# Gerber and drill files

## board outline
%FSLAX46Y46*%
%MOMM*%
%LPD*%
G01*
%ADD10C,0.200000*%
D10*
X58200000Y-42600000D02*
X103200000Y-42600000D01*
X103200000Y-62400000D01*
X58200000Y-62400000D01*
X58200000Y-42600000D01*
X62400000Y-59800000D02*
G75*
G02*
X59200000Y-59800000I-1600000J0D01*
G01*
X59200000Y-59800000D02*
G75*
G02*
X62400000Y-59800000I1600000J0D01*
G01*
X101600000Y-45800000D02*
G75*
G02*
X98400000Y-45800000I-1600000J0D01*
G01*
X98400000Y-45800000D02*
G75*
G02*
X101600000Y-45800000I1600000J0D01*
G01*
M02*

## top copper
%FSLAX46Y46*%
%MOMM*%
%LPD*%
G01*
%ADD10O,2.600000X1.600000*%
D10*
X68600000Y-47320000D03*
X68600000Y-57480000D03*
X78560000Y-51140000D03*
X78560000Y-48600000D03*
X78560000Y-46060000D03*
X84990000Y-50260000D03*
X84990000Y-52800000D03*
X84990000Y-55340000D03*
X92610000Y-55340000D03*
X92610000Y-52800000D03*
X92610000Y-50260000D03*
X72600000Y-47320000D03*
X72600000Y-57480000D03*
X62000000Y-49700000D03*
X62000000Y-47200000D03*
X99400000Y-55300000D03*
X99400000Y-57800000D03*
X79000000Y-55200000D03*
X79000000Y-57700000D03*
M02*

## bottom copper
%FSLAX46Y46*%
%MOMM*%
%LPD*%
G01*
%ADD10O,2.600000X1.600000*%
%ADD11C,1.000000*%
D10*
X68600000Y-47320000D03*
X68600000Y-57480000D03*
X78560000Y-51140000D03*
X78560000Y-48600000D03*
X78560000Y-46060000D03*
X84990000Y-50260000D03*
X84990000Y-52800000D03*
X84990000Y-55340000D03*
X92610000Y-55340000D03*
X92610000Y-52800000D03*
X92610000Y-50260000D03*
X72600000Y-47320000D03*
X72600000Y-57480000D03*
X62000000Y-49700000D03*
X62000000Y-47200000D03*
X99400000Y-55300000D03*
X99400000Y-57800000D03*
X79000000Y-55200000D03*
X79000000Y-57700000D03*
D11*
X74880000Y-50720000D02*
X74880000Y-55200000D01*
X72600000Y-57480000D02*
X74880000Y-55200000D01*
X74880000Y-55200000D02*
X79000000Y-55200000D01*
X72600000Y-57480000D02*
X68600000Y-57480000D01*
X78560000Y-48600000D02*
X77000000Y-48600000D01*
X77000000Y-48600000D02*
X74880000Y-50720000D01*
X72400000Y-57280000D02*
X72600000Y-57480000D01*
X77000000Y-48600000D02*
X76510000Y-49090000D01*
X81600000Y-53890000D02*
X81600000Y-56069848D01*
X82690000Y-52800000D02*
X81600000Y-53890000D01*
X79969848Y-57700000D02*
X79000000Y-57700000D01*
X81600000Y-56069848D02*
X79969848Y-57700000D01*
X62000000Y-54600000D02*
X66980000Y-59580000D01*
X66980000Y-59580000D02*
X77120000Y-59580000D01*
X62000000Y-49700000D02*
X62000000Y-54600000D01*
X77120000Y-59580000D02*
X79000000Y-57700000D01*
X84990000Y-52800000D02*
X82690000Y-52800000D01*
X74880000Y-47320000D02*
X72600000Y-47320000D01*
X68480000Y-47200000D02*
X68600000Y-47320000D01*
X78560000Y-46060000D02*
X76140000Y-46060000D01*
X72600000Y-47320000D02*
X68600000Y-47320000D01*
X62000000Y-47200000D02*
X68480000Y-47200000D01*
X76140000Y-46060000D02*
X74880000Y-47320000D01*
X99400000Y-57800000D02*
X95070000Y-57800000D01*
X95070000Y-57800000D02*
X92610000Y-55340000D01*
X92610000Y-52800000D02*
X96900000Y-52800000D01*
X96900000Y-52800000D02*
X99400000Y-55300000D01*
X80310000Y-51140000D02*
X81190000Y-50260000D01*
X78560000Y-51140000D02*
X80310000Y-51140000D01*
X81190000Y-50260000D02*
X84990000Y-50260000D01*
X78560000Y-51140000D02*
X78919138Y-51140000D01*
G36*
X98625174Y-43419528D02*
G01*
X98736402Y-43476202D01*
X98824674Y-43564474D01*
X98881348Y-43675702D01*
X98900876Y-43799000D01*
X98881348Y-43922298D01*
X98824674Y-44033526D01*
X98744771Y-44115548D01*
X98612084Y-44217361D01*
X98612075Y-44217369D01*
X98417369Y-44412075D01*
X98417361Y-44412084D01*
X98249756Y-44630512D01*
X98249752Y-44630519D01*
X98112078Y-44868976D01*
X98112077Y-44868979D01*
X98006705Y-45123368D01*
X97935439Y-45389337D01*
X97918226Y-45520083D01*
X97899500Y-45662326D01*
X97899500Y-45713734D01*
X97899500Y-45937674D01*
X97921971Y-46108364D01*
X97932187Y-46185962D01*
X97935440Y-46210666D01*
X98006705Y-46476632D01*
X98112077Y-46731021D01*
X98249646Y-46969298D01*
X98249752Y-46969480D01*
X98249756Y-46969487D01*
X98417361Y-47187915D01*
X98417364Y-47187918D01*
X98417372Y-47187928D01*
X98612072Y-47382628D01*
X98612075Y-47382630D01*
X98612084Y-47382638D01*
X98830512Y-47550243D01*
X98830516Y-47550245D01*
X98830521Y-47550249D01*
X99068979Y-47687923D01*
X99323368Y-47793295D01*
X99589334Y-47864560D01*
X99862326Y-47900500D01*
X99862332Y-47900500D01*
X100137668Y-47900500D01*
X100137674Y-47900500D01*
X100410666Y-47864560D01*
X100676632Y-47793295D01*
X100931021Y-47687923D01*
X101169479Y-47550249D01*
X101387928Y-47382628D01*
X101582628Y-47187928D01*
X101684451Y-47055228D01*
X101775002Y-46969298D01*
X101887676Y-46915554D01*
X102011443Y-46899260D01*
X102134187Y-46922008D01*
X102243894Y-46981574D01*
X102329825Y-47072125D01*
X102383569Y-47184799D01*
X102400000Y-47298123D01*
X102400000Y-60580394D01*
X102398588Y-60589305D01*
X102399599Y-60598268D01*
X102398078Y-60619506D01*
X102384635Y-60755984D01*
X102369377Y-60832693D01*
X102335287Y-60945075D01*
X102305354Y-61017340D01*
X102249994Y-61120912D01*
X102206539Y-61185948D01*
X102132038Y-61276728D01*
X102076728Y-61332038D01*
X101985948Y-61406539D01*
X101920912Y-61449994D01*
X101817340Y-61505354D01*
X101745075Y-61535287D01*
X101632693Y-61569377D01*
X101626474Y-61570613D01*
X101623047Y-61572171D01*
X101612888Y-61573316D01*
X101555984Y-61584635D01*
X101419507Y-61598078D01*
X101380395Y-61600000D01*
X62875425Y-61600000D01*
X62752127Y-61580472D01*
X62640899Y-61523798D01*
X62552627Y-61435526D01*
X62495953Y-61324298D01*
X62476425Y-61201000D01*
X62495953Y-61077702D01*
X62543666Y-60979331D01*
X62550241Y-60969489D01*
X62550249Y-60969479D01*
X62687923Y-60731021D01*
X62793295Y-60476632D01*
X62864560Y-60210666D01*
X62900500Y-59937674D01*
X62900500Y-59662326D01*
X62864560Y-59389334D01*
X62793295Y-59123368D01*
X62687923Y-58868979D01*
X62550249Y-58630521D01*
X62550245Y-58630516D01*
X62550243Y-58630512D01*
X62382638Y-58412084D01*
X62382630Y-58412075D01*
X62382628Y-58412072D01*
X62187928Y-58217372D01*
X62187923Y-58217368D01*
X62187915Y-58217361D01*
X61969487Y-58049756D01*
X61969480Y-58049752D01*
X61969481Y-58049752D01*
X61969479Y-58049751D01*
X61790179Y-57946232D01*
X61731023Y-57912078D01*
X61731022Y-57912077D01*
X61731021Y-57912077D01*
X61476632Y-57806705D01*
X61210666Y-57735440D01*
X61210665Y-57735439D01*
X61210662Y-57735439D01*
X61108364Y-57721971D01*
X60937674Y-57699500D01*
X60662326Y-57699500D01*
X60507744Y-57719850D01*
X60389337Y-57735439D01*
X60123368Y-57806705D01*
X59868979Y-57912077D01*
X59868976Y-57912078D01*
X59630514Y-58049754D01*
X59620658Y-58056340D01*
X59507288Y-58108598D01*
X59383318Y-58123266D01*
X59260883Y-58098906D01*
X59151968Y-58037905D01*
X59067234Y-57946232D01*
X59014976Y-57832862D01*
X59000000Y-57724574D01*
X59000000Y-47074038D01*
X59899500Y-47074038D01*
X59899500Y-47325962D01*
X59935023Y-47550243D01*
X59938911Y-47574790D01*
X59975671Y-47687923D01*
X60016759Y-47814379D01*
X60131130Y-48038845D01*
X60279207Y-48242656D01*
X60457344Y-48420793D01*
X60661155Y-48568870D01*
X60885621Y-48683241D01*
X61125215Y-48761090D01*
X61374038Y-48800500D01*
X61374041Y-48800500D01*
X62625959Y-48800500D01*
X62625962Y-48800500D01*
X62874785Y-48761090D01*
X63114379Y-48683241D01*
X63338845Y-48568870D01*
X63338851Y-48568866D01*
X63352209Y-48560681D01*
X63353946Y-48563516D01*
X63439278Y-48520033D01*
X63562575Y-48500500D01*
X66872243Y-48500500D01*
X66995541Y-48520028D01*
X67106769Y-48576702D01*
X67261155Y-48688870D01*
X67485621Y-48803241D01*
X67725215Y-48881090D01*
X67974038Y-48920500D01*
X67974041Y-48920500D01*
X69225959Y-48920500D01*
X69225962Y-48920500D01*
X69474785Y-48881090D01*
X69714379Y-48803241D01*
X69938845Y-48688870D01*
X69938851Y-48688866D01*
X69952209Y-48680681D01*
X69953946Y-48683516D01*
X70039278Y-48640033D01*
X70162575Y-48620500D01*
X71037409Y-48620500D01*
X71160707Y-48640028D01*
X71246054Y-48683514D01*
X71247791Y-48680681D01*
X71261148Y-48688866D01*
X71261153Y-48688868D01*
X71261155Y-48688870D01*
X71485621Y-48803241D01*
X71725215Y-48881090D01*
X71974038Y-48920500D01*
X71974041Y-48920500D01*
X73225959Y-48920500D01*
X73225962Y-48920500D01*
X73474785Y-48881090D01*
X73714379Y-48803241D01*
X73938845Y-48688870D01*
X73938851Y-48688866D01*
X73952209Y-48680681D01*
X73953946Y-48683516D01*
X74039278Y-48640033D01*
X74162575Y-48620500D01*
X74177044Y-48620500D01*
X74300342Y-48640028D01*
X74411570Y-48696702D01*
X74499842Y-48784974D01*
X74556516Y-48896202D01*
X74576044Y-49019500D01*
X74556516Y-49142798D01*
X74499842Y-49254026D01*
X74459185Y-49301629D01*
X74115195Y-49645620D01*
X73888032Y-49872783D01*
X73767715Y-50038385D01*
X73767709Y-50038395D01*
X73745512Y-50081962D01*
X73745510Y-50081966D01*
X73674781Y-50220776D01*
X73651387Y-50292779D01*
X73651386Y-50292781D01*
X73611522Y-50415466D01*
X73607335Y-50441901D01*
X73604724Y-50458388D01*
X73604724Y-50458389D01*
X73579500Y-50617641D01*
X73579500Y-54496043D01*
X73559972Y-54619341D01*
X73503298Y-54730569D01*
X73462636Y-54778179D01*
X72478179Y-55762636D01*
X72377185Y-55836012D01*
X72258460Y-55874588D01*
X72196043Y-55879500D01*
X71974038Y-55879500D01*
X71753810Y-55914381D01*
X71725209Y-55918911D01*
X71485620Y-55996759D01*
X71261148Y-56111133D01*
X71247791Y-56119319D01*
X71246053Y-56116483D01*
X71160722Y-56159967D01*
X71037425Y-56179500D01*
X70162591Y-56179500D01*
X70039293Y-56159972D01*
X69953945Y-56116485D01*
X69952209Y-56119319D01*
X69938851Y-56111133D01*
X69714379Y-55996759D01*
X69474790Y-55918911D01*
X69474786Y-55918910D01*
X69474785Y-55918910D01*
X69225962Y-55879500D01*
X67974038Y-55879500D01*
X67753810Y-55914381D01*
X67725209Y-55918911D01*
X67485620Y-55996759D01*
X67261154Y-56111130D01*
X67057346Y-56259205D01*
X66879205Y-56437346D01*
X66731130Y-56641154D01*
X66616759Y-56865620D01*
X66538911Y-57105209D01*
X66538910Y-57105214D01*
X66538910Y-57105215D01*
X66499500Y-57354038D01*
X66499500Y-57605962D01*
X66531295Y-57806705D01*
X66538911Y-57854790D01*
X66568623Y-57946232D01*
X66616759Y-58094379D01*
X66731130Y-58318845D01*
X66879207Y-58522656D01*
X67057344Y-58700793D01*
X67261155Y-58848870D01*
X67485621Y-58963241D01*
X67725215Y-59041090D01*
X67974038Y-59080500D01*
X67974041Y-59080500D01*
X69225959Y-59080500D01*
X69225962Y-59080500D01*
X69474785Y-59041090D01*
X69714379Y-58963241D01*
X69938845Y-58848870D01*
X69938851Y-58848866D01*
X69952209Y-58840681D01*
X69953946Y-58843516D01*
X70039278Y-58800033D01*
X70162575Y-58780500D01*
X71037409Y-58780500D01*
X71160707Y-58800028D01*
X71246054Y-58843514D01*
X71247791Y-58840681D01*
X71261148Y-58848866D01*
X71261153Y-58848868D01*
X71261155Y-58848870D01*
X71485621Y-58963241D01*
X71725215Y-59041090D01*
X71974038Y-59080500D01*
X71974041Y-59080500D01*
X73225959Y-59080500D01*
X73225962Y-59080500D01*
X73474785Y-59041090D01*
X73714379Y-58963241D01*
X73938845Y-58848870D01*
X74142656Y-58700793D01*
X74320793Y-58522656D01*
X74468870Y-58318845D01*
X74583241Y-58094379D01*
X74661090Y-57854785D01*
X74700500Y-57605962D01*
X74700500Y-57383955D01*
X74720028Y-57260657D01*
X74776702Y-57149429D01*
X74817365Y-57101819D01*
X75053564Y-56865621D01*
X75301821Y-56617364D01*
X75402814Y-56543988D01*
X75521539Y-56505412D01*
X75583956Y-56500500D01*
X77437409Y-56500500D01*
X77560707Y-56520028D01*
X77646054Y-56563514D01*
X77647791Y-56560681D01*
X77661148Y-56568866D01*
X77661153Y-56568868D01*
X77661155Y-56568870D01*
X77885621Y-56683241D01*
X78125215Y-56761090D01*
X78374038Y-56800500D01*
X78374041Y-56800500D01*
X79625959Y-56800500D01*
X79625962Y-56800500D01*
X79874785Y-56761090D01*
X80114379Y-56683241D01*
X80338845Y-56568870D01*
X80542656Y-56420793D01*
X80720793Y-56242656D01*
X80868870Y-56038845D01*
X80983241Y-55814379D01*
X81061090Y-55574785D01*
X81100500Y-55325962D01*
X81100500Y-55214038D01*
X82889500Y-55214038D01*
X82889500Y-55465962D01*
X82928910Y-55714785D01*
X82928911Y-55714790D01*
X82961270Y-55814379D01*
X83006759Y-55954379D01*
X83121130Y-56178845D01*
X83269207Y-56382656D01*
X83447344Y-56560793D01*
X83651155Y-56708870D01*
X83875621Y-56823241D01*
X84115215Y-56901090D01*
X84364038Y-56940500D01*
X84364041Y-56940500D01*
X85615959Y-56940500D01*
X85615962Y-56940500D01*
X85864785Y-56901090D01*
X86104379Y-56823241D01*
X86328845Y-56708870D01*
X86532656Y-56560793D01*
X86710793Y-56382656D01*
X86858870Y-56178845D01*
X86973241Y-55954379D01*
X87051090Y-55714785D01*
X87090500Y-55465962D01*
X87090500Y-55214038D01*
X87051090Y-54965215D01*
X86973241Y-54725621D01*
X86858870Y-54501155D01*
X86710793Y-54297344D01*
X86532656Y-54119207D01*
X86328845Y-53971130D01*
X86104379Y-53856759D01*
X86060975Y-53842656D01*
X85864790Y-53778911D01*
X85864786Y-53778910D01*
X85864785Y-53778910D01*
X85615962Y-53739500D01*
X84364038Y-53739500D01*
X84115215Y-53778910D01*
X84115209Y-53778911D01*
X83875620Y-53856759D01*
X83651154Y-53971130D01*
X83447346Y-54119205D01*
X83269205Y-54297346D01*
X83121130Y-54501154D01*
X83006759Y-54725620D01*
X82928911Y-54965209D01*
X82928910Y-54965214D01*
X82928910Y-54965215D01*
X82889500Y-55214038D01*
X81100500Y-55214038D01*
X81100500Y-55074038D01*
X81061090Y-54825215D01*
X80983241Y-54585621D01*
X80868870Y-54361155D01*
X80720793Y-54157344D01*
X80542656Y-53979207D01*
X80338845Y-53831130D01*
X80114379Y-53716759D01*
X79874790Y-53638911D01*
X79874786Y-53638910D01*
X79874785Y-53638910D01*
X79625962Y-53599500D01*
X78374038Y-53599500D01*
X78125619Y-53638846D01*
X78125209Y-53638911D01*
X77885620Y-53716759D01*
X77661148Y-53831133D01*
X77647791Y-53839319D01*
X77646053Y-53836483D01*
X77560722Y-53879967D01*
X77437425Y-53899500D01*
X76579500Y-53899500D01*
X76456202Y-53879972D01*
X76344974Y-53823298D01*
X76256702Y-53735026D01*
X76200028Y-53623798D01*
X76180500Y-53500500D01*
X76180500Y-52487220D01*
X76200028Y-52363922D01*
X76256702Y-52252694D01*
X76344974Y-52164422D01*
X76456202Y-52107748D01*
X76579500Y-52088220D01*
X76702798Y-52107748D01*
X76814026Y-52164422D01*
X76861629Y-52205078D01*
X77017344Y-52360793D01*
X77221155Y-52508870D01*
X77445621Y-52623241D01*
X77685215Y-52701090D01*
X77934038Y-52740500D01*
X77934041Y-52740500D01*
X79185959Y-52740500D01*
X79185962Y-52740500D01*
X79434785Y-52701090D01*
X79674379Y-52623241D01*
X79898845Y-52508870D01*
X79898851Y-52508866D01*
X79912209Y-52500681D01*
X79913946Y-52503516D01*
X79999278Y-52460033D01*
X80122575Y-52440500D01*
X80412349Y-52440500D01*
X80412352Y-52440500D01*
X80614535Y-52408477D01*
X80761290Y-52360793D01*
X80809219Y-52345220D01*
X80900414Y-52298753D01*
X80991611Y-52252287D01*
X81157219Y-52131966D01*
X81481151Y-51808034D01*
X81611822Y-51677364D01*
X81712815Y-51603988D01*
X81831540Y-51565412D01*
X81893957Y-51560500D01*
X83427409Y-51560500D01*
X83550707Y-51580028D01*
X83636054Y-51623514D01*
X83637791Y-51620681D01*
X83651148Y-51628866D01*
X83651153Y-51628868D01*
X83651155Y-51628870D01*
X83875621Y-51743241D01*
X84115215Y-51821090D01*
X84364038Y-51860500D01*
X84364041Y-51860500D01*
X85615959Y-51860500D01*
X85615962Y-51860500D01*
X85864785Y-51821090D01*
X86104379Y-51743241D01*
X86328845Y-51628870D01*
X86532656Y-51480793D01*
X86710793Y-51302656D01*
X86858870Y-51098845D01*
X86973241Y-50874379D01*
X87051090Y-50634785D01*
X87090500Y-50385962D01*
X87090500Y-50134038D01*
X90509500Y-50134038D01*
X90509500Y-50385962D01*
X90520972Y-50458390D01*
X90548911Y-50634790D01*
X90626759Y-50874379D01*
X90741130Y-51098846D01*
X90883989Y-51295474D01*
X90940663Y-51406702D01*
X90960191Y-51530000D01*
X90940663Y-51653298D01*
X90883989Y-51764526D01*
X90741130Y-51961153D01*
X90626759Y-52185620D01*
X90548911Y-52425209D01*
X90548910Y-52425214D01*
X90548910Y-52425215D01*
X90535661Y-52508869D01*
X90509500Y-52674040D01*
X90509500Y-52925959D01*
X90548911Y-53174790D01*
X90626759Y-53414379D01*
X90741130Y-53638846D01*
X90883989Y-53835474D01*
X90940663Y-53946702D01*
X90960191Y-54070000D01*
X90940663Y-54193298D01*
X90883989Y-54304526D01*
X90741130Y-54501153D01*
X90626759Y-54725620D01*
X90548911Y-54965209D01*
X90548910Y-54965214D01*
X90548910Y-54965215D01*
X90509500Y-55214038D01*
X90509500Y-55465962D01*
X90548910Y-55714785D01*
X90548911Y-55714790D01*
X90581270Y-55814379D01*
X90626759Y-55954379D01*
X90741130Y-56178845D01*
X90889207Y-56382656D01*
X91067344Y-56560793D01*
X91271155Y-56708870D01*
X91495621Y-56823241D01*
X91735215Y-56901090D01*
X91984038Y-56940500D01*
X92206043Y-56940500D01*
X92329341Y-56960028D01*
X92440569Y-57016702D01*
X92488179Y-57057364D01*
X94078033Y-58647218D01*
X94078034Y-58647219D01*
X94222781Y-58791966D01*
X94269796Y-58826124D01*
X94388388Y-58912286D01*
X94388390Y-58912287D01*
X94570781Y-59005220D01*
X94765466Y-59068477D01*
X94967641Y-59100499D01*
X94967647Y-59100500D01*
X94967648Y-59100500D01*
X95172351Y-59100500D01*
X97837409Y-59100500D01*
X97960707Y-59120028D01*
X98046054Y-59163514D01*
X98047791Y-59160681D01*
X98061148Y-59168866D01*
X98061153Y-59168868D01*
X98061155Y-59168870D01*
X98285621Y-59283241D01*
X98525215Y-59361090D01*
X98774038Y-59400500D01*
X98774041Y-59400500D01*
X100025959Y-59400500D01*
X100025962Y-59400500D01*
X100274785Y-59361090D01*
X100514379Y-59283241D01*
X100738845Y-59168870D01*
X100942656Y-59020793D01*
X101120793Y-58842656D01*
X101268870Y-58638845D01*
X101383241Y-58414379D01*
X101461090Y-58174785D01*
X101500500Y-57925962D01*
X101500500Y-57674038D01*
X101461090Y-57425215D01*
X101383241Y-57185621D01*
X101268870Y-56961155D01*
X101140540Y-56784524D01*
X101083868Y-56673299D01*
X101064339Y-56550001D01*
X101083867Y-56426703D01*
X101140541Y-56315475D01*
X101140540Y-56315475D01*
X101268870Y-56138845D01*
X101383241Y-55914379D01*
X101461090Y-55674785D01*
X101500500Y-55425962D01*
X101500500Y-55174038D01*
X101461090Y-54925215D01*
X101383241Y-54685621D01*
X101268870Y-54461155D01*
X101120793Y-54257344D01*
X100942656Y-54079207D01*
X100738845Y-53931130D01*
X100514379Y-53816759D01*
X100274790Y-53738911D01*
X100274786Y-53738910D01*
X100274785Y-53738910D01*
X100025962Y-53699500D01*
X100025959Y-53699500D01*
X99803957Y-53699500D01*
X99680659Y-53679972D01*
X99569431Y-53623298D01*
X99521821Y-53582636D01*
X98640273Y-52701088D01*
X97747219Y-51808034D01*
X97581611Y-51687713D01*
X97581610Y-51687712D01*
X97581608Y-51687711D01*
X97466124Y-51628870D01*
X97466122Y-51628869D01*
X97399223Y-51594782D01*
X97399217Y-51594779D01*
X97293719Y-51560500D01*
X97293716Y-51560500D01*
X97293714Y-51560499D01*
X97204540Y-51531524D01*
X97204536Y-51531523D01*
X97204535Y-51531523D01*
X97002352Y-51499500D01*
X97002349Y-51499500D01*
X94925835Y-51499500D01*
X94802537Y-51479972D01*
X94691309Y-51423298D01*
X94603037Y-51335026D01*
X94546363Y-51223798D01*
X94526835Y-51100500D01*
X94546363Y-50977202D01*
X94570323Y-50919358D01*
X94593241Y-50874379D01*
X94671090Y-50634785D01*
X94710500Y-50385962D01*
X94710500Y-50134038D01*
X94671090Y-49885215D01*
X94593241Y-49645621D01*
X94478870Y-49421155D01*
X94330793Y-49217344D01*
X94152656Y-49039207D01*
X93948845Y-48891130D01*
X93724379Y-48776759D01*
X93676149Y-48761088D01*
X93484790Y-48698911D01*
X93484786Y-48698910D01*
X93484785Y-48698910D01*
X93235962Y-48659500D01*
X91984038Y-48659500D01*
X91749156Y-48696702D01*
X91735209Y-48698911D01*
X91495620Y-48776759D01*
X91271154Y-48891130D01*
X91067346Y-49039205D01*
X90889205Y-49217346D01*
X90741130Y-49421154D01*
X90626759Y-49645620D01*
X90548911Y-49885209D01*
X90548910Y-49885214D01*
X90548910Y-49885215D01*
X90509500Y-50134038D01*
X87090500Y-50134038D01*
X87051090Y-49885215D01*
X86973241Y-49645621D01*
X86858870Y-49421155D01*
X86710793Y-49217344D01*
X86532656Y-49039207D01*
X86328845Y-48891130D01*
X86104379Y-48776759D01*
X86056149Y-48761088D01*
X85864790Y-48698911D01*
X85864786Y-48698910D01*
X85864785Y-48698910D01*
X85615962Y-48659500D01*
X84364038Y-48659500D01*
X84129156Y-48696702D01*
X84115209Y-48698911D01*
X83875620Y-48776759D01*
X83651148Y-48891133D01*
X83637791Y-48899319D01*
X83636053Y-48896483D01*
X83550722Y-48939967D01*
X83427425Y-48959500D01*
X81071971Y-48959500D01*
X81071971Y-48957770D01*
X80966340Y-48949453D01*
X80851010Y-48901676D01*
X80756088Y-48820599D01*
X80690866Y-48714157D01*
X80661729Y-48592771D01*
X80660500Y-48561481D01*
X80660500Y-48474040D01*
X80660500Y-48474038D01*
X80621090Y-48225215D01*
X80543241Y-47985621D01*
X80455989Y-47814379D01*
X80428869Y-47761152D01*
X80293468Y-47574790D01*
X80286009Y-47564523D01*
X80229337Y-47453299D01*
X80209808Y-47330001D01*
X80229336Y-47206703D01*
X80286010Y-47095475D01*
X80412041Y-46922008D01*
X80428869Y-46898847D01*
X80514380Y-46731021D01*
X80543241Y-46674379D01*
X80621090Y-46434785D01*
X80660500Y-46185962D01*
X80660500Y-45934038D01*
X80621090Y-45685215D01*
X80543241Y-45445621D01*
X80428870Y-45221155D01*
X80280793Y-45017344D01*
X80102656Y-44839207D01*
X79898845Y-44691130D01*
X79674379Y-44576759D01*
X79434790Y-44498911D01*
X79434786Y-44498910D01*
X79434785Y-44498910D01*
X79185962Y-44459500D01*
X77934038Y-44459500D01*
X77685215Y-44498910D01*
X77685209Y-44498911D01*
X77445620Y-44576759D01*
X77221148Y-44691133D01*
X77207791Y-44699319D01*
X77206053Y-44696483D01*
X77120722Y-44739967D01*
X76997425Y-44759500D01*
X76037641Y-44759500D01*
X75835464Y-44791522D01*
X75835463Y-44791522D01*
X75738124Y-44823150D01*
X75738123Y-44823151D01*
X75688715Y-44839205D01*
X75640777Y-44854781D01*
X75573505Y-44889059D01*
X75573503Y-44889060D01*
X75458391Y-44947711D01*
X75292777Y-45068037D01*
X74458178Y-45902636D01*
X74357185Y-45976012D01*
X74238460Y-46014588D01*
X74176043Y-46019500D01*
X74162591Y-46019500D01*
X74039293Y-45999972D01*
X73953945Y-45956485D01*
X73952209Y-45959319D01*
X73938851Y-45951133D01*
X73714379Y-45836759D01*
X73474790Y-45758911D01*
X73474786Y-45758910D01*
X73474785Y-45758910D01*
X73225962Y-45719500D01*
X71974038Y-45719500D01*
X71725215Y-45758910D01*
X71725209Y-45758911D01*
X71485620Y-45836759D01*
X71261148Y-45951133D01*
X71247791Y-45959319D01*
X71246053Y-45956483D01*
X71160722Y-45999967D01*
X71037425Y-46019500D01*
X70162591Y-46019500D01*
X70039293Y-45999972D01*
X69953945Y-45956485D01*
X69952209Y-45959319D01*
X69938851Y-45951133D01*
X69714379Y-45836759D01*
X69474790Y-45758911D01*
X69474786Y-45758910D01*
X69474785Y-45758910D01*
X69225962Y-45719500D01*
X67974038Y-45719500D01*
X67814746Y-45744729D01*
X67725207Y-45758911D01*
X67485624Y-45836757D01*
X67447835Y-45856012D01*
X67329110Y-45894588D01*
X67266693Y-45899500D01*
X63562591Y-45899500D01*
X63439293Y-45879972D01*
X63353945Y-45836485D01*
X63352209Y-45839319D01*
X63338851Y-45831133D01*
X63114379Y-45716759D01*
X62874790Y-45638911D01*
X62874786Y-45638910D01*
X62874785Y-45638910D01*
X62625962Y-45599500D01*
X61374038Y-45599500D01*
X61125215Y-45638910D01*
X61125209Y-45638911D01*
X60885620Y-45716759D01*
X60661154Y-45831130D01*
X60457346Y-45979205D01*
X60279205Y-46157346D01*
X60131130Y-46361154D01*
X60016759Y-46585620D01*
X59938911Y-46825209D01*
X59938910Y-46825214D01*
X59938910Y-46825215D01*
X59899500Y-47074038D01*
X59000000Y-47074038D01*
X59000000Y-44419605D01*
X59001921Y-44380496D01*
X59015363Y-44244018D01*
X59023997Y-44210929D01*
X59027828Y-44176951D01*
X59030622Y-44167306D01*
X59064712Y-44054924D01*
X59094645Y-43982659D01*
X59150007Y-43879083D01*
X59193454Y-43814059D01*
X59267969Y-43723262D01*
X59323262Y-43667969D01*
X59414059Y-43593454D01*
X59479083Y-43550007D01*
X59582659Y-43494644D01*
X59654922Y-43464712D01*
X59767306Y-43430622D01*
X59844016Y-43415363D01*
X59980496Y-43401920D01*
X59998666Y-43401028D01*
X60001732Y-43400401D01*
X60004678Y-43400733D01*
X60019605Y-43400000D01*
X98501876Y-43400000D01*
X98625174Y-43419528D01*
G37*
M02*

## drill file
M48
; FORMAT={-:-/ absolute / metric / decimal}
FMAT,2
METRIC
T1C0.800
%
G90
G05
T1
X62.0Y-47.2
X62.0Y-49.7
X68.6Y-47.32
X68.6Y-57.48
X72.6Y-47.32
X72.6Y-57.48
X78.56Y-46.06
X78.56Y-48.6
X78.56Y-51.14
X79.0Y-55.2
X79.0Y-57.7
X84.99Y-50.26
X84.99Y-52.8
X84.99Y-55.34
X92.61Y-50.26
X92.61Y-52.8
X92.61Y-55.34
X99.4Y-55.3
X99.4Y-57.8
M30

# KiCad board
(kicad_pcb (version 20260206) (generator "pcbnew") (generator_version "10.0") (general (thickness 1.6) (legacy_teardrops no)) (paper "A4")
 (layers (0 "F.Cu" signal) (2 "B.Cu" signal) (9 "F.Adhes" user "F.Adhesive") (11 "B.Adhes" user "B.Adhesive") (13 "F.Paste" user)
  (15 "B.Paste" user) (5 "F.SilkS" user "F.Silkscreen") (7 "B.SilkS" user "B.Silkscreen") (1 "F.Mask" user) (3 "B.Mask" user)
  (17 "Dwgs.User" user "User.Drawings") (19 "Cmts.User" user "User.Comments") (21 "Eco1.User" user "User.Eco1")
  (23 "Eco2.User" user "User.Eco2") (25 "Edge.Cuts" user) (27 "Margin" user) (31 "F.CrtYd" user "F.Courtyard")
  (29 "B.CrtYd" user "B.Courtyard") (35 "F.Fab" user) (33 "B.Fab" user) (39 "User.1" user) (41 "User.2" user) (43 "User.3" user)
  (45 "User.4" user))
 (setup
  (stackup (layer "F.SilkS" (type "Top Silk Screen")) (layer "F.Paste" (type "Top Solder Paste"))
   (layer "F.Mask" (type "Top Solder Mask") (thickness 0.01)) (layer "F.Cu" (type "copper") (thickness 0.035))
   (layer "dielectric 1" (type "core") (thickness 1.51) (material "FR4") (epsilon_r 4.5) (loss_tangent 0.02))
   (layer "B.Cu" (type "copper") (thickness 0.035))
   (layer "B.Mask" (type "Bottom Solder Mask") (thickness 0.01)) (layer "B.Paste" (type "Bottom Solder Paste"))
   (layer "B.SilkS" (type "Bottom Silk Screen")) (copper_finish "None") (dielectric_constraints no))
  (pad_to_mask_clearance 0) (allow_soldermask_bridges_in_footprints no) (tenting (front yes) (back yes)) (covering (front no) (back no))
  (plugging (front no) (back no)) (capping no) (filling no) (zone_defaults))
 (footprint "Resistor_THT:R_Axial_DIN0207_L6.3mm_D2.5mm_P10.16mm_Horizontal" (layer "F.Cu") (at 68.6 47.32 -90)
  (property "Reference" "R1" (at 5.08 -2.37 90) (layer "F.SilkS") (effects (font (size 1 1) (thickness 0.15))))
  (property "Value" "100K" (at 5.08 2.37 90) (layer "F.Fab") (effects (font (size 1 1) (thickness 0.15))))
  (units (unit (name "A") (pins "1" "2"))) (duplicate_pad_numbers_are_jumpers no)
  (pad "1" thru_hole oval (at 0 0) (size 2.6 1.6) (drill 0.8) (layers "*.Cu" "*.Mask") (remove_unused_layers no) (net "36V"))
  (pad "2" thru_hole oval (at 10.16 0) (size 2.6 1.6) (drill 0.8) (layers "*.Cu" "*.Mask") (remove_unused_layers no) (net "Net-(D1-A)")))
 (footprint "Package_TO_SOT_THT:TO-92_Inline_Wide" (layer "F.Cu") (at 78.56 51.14 90)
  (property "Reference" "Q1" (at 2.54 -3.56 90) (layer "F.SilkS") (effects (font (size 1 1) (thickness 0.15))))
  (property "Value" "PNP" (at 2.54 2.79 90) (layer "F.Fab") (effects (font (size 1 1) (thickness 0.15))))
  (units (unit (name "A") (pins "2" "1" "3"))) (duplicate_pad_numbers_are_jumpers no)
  (pad "1" thru_hole oval (at 0 0 90) (size 1.6 2.6) (drill 0.8) (layers "*.Cu" "*.Mask") (remove_unused_layers no) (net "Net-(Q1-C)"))
  (pad "2" thru_hole oval (at 2.54 0 90) (size 1.6 2.6) (drill 0.8) (layers "*.Cu" "*.Mask") (remove_unused_layers no) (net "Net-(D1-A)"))
  (pad "3" thru_hole oval (at 5.08 0 90) (size 1.6 2.6) (drill 0.8) (layers "*.Cu" "*.Mask") (remove_unused_layers no) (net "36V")))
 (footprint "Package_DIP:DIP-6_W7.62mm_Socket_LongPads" (layer "F.Cu") (at 84.99 50.26)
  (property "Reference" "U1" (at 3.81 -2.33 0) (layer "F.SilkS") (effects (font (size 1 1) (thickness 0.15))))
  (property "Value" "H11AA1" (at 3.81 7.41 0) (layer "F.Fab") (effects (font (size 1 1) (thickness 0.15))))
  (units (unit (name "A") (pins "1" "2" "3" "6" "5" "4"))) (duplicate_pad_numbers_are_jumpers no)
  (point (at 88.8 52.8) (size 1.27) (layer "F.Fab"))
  (pad "1" thru_hole oval (at 0 0) (size 2.6 1.6) (drill 0.8) (layers "*.Cu" "*.Mask") (remove_unused_layers no) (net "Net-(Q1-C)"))
  (pad "2" thru_hole oval (at 0 2.54) (size 2.6 1.6) (drill 0.8) (layers "*.Cu" "*.Mask") (remove_unused_layers no) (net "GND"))
  (pad "3" thru_hole oval (at 0 5.08) (size 2.6 1.6) (drill 0.8) (layers "*.Cu" "*.Mask") (remove_unused_layers no)
   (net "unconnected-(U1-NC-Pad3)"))
  (pad "4" thru_hole oval (at 7.62 5.08) (size 2.6 1.6) (drill 0.8) (layers "*.Cu" "*.Mask") (remove_unused_layers no)
   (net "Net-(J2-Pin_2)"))
  (pad "5" thru_hole oval (at 7.62 2.54) (size 2.6 1.6) (drill 0.8) (layers "*.Cu" "*.Mask") (remove_unused_layers no)
   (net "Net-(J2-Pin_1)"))
  (pad "6" thru_hole oval (at 7.62 0) (size 2.6 1.6) (drill 0.8) (layers "*.Cu" "*.Mask") (remove_unused_layers no)
   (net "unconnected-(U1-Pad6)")))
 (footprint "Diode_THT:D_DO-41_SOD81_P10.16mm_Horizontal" (layer "F.Cu") (at 72.6 47.32 -90)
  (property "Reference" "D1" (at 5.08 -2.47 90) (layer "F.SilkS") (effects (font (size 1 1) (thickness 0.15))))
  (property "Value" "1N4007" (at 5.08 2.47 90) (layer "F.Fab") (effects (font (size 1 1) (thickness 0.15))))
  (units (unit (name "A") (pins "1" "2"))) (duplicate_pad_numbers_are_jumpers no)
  (pad "1" thru_hole oval (at 0 0) (size 2.6 1.6) (drill 0.8) (layers "*.Cu" "*.Mask") (remove_unused_layers no) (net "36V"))
  (pad "2" thru_hole oval (at 10.16 0) (size 2.6 1.6) (drill 0.8) (layers "*.Cu" "*.Mask") (remove_unused_layers no) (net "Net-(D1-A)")))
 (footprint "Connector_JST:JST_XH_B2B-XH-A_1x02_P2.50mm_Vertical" (layer "F.Cu") (at 62 49.7 90)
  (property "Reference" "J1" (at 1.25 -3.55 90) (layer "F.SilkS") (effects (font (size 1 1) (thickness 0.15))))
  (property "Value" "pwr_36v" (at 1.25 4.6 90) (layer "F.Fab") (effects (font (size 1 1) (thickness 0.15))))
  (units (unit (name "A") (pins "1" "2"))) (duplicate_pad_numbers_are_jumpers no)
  (pad "1" thru_hole oval (at 0 0 180) (size 2.6 1.6) (drill 0.8) (layers "*.Cu" "*.Mask") (remove_unused_layers no) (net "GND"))
  (pad "2" thru_hole oval (at 2.5 0 180) (size 2.6 1.6) (drill 0.8) (layers "*.Cu" "*.Mask") (remove_unused_layers no) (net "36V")))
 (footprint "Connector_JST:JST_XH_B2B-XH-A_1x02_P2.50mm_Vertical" (layer "F.Cu") (at 99.4 55.3 -90)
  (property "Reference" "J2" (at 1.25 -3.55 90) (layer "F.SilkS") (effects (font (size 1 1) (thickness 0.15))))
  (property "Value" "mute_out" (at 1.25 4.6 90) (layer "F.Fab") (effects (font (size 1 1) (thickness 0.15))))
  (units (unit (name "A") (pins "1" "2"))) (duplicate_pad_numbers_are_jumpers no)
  (pad "1" thru_hole oval (at 0 0) (size 2.6 1.6) (drill 0.8) (layers "*.Cu" "*.Mask") (remove_unused_layers no) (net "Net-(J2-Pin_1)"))
  (pad "2" thru_hole oval (at 2.5 0) (size 2.6 1.6) (drill 0.8) (layers "*.Cu" "*.Mask") (remove_unused_layers no) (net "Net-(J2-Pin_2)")))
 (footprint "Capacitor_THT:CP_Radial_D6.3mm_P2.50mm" (layer "F.Cu") (at 79 55.2 -90)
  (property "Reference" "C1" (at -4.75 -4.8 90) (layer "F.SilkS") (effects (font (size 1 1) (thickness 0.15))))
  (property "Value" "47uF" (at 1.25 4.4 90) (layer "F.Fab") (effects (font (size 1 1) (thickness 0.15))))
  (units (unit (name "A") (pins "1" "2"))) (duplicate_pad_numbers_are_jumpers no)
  (pad "1" thru_hole oval (at 0 0 270) (size 1.6 2.6) (drill 0.8) (layers "*.Cu" "*.Mask") (remove_unused_layers no) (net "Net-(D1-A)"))
  (pad "2" thru_hole oval (at 2.5 0 270) (size 1.6 2.6) (drill 0.8) (layers "*.Cu" "*.Mask") (remove_unused_layers no) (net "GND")))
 (gr_rect (start 58.2 42.6) (end 103.2 62.4) (stroke (width 0.2) (type solid)) (fill no) (layer "Edge.Cuts"))
 (gr_circle (center 60.8 59.8) (end 62.4 59.8) (stroke (width 0.2) (type solid)) (fill no) (layer "Edge.Cuts"))
 (gr_circle (center 100 45.8) (end 101.6 45.8) (stroke (width 0.2) (type solid)) (fill no) (layer "Edge.Cuts"))
 (segment (start 74.88 50.72) (end 74.88 55.2) (width 1) (layer "B.Cu") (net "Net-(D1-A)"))
 (segment (start 72.6 57.48) (end 74.88 55.2) (width 1) (layer "B.Cu") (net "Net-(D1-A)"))
 (segment (start 74.88 55.2) (end 79 55.2) (width 1) (layer "B.Cu") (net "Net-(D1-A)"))
 (segment (start 72.6 57.48) (end 68.6 57.48) (width 1) (layer "B.Cu") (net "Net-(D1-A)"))
 (segment (start 78.56 48.6) (end 77 48.6) (width 1) (layer "B.Cu") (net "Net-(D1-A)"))
 (segment (start 77 48.6) (end 74.88 50.72) (width 1) (layer "B.Cu") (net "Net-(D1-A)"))
 (segment (start 72.4 57.28) (end 72.6 57.48) (width 1) (layer "B.Cu") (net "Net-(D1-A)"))
 (segment (start 77 48.6) (end 76.51 49.09) (width 1) (layer "B.Cu") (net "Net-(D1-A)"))
 (segment (start 81.6 53.89) (end 81.6 56.069848) (width 1) (layer "B.Cu") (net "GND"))
 (segment (start 82.69 52.8) (end 81.6 53.89) (width 1) (layer "B.Cu") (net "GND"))
 (segment (start 79.969848 57.7) (end 79 57.7) (width 1) (layer "B.Cu") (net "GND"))
 (segment (start 81.6 56.069848) (end 79.969848 57.7) (width 1) (layer "B.Cu") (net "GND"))
 (segment (start 62 54.6) (end 66.98 59.58) (width 1) (layer "B.Cu") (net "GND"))
 (segment (start 66.98 59.58) (end 77.12 59.58) (width 1) (layer "B.Cu") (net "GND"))
 (segment (start 62 49.7) (end 62 54.6) (width 1) (layer "B.Cu") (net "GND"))
 (segment (start 77.12 59.58) (end 79 57.7) (width 1) (layer "B.Cu") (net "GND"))
 (segment (start 84.99 52.8) (end 82.69 52.8) (width 1) (layer "B.Cu") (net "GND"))
 (segment (start 74.88 47.32) (end 72.6 47.32) (width 1) (layer "B.Cu") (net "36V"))
 (segment (start 68.48 47.2) (end 68.6 47.32) (width 1) (layer "B.Cu") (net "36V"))
 (segment (start 78.56 46.06) (end 76.14 46.06) (width 1) (layer "B.Cu") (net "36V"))
 (segment (start 72.6 47.32) (end 68.6 47.32) (width 1) (layer "B.Cu") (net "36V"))
 (segment (start 62 47.2) (end 68.48 47.2) (width 1) (layer "B.Cu") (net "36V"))
 (segment (start 76.14 46.06) (end 74.88 47.32) (width 1) (layer "B.Cu") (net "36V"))
 (segment (start 99.4 57.8) (end 95.07 57.8) (width 1) (layer "B.Cu") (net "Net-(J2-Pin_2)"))
 (segment (start 95.07 57.8) (end 92.61 55.34) (width 1) (layer "B.Cu") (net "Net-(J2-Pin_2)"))
 (segment (start 92.61 52.8) (end 96.9 52.8) (width 1) (layer "B.Cu") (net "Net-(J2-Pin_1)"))
 (segment (start 96.9 52.8) (end 99.4 55.3) (width 1) (layer "B.Cu") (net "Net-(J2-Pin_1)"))
 (segment (start 80.31 51.14) (end 81.19 50.26) (width 1) (layer "B.Cu") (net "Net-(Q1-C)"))
 (segment (start 78.56 51.14) (end 80.31 51.14) (width 1) (layer "B.Cu") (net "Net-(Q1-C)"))
 (segment (start 81.19 50.26) (end 84.99 50.26) (width 1) (layer "B.Cu") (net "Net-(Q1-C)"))
 (segment (start 78.56 51.14) (end 78.919138 51.14) (width 1) (layer "B.Cu") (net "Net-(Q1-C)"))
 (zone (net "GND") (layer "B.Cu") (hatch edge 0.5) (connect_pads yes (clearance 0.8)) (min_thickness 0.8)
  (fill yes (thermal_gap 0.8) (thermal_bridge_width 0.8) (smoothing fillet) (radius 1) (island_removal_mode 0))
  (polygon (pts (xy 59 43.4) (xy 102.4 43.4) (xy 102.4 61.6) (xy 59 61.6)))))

